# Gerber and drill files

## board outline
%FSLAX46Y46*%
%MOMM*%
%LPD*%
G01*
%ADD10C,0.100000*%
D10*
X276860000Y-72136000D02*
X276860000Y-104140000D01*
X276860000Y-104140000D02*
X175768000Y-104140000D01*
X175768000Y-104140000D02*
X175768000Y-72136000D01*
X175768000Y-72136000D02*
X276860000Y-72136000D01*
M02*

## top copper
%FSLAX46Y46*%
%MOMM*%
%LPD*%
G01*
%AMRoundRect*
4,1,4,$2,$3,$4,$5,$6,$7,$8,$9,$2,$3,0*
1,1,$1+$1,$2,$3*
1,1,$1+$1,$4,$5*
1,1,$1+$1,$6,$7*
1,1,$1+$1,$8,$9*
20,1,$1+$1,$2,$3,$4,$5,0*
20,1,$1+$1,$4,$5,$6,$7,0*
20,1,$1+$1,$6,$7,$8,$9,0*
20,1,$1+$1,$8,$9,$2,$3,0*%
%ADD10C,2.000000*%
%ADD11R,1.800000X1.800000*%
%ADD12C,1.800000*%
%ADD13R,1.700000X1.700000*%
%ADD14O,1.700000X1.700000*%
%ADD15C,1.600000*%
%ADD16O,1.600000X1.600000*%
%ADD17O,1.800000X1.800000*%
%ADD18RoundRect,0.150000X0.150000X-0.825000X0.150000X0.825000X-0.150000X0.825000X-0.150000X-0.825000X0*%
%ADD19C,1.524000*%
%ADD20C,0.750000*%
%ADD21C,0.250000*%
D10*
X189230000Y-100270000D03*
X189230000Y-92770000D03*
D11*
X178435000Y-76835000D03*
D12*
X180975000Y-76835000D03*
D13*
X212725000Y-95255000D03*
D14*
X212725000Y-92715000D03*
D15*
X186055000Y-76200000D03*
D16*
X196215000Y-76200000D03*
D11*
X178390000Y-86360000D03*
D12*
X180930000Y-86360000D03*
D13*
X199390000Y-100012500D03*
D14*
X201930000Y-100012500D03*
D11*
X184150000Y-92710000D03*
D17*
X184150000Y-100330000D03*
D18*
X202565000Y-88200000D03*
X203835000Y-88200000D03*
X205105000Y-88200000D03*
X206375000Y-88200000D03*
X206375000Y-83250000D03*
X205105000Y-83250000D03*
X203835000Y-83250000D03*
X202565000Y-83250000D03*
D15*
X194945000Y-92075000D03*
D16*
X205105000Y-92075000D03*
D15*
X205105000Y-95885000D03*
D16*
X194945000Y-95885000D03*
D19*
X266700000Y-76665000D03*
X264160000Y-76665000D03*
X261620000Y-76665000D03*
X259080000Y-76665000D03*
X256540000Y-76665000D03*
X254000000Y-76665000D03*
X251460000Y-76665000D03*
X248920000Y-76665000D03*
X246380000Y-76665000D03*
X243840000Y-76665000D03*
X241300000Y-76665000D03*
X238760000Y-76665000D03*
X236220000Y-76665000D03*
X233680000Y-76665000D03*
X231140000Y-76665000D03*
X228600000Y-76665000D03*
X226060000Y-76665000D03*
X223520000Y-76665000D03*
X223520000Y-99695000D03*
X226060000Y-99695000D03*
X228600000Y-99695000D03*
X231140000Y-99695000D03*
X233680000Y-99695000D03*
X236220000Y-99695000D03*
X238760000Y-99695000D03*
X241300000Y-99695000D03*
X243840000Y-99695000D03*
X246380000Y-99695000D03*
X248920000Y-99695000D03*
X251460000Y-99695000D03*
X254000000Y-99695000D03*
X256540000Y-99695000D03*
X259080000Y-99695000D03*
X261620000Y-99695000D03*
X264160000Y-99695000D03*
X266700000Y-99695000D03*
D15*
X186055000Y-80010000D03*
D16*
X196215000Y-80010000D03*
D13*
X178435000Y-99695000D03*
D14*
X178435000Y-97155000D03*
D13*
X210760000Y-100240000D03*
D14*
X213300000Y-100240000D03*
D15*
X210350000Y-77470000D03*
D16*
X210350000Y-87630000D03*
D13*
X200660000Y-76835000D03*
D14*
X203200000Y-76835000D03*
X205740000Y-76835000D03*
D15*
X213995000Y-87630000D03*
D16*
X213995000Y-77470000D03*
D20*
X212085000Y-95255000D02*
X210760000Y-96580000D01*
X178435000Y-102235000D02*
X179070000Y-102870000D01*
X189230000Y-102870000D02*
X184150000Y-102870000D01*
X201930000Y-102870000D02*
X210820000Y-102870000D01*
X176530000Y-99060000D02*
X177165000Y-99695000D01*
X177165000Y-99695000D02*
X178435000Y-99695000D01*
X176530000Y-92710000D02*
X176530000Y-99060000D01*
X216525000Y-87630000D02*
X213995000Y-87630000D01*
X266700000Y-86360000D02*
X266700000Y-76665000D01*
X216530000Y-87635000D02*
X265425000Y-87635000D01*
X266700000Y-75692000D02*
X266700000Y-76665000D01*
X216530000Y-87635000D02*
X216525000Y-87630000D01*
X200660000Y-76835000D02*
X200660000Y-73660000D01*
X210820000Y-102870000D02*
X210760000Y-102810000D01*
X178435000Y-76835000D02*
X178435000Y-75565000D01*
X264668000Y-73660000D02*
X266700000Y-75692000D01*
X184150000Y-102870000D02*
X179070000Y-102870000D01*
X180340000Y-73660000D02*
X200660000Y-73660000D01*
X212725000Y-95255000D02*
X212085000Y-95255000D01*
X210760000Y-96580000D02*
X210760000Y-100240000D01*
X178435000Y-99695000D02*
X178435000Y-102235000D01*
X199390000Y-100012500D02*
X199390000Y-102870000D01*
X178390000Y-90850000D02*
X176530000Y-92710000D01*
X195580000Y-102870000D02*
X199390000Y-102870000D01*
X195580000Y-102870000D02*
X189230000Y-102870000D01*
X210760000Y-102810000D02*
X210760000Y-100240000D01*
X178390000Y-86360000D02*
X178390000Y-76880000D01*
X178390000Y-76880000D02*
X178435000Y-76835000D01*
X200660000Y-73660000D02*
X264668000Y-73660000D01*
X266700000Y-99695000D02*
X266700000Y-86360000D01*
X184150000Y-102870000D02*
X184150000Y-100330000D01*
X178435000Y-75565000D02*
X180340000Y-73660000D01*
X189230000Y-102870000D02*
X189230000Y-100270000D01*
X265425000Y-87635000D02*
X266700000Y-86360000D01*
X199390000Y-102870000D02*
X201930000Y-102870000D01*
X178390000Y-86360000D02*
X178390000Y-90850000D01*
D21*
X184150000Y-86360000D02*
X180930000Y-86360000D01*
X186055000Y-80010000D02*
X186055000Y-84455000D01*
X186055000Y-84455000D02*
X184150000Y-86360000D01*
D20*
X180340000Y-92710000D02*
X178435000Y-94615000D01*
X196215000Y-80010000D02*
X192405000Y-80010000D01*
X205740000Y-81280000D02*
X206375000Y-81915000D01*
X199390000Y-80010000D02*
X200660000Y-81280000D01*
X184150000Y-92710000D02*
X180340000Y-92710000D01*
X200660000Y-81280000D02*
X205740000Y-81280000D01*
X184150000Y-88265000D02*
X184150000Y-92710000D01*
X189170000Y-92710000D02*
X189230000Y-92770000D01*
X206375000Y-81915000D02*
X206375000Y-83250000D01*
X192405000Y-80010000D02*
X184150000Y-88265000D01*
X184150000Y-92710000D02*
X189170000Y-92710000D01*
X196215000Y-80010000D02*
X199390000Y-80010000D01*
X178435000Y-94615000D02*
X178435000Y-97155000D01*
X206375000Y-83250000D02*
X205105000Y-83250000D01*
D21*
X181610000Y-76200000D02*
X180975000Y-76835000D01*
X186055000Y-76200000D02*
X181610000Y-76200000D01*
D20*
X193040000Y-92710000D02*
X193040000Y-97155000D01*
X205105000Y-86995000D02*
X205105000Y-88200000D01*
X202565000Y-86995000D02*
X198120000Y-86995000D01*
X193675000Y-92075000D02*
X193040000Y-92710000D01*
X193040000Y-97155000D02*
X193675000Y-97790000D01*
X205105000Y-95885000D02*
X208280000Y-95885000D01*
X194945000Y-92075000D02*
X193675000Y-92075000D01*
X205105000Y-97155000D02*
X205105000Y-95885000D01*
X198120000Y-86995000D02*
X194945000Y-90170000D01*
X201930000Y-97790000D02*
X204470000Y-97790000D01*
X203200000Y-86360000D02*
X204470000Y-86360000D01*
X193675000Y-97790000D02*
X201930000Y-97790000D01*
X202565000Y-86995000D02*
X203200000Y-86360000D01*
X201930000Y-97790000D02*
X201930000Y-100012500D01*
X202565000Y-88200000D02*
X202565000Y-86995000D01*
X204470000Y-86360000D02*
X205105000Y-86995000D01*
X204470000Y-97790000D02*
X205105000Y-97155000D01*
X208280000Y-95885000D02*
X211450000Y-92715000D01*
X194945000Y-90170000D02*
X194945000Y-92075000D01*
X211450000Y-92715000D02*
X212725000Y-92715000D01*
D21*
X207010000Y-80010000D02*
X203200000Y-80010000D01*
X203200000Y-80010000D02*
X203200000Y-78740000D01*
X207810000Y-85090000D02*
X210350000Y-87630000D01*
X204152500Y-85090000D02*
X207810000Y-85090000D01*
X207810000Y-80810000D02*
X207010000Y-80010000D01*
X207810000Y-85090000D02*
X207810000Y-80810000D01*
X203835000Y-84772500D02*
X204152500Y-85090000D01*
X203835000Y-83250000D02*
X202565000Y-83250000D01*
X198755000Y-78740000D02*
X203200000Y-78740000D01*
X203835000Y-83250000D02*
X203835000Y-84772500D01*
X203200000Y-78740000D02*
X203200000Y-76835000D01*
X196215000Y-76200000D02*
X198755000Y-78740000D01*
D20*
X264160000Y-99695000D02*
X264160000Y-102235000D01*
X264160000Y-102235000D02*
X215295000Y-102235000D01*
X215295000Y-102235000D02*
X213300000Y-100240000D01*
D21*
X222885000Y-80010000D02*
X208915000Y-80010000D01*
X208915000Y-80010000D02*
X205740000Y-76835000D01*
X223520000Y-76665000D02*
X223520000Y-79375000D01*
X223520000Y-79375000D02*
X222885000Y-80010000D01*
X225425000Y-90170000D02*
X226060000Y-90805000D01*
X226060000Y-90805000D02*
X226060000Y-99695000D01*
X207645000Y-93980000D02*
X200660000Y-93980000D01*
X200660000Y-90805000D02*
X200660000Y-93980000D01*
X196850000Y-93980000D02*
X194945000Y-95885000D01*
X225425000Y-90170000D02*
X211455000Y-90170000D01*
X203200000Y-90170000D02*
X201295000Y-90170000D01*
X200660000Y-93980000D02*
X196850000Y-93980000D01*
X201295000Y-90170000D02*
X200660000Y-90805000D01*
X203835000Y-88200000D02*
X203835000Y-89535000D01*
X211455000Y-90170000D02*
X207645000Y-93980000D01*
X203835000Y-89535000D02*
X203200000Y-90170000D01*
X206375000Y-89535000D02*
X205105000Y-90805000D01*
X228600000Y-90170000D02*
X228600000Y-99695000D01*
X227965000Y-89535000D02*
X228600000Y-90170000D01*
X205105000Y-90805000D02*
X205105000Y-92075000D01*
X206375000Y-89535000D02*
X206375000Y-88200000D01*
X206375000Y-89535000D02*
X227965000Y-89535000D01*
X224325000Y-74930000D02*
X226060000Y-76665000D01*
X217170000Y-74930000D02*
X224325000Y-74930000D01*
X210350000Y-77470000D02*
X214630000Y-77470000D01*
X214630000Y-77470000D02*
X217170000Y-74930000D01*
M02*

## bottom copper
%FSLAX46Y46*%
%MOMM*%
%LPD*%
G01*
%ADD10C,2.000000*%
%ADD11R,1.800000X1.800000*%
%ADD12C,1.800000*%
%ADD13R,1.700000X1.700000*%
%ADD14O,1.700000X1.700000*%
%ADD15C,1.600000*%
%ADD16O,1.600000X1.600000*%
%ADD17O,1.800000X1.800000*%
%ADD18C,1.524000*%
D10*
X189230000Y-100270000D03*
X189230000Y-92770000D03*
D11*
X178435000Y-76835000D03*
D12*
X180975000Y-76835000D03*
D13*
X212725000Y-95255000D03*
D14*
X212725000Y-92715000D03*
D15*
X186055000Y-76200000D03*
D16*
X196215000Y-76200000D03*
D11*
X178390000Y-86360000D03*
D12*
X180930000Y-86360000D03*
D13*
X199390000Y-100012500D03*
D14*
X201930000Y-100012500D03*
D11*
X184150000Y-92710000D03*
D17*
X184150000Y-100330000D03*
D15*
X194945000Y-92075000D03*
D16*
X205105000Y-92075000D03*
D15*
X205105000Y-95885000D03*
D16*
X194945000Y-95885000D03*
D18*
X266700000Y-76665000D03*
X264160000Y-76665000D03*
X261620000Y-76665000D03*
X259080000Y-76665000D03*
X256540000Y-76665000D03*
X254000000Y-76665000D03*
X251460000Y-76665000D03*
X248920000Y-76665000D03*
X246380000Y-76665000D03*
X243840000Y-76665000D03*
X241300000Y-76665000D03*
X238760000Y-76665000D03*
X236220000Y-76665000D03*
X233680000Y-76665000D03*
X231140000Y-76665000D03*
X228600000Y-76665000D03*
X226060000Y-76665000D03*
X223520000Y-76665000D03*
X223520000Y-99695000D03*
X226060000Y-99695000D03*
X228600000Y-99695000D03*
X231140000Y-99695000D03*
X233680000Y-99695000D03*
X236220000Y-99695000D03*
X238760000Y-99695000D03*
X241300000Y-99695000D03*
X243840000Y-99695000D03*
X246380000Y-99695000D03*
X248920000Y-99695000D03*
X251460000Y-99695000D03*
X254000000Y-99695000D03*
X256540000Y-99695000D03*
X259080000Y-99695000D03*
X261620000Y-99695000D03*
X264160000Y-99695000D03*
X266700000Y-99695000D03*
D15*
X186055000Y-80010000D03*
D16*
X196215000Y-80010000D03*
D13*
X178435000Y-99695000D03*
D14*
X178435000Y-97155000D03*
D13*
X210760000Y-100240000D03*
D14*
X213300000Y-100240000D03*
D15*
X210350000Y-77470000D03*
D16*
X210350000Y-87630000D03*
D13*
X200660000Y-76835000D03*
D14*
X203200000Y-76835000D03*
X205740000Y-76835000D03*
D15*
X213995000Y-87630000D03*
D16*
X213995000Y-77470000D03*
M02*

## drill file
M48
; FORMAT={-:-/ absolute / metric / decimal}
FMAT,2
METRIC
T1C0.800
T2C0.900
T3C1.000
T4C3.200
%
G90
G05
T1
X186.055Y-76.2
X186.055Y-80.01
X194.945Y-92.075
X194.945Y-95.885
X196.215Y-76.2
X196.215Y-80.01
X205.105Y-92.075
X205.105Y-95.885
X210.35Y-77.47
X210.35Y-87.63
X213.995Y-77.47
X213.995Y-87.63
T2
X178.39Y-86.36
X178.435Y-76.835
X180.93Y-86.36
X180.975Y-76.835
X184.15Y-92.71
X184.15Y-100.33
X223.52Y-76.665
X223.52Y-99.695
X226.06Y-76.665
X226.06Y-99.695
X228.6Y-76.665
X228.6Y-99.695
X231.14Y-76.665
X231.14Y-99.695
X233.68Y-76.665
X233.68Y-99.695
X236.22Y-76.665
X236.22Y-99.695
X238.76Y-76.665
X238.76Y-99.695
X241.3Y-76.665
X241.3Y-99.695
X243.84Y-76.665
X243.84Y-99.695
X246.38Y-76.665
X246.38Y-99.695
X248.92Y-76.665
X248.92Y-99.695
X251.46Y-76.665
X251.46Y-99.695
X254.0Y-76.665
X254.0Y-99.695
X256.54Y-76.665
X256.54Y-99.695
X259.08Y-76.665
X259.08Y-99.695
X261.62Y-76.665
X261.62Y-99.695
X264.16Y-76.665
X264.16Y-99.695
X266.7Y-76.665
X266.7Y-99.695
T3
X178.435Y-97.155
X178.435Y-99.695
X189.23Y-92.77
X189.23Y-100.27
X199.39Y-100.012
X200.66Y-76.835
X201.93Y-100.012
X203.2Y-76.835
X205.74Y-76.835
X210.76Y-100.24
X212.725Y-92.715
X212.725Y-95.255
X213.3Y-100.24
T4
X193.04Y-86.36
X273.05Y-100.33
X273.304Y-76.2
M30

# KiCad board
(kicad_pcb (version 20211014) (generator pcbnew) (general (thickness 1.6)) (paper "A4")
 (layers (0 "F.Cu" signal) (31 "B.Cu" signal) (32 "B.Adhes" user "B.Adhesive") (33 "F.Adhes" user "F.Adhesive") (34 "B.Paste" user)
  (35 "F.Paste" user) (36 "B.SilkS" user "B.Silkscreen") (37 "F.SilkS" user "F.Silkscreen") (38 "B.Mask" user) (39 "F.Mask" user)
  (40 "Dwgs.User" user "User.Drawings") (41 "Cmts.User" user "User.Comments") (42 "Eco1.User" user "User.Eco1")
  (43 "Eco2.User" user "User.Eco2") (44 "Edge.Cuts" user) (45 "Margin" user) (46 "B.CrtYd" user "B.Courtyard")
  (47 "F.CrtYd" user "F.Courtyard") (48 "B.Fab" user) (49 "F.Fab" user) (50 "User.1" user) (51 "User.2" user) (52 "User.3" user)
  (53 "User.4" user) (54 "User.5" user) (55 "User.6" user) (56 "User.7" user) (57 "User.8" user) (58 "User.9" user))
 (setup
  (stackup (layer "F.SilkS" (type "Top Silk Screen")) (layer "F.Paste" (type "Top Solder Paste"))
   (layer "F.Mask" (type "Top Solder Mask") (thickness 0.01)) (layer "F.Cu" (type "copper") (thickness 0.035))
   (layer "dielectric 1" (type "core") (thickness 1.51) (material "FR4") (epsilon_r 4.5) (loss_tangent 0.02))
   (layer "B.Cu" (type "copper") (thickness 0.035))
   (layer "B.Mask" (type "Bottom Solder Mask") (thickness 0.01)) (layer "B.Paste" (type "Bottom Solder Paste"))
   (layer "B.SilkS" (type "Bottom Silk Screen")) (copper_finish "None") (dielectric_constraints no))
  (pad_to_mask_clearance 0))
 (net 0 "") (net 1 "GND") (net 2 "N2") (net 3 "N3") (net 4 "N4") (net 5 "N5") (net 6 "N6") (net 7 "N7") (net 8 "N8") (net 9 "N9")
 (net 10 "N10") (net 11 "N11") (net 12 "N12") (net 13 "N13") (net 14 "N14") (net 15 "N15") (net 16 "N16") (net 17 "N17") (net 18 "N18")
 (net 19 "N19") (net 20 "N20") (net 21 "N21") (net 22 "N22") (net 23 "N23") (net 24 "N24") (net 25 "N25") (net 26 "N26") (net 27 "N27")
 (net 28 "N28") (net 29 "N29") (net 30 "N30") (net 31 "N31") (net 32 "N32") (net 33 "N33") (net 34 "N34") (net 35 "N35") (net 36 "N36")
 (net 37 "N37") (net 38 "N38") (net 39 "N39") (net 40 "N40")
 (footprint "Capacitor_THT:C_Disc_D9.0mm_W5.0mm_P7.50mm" (layer "F.Cu") (at 189.23 100.27 90)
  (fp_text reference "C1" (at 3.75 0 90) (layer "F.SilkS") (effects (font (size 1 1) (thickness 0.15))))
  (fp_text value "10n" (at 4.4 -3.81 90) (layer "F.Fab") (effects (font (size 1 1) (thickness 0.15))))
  (pad "1" thru_hole circle (at 0 0 90) (size 2 2) (drill 1) (layers *.Cu *.Mask) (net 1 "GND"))
  (pad "2" thru_hole circle (at 7.5 0 90) (size 2 2) (drill 1) (layers *.Cu *.Mask) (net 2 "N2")))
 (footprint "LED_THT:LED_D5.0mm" (layer "F.Cu") (at 178.435 76.835)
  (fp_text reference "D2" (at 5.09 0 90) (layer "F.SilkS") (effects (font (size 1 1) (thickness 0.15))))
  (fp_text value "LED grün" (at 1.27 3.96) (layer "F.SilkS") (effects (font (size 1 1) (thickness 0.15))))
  (pad "1" thru_hole rect (at 0 0) (size 1.8 1.8) (drill 0.9) (layers *.Cu *.Mask) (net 1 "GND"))
  (pad "2" thru_hole circle (at 2.54 0) (size 1.8 1.8) (drill 0.9) (layers *.Cu *.Mask) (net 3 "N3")))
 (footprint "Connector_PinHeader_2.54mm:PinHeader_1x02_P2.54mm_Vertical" (layer "F.Cu") (at 212.725 95.255 180)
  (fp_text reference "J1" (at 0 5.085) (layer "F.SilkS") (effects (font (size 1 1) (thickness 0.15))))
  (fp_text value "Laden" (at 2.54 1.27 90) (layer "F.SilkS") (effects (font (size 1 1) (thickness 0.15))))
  (pad "1" thru_hole rect (at 0 0 180) (size 1.7 1.7) (drill 1) (layers *.Cu *.Mask) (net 1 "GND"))
  (pad "2" thru_hole oval (at 0 2.54 180) (size 1.7 1.7) (drill 1) (layers *.Cu *.Mask) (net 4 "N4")))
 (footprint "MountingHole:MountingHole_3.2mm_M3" (layer "F.Cu") (at 193.04 86.36)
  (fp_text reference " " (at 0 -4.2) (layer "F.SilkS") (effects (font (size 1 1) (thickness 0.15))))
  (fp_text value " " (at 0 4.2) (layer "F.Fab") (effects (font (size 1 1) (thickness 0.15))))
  (pad "" np_thru_hole circle (at 0 0) (size 3.2 3.2) (drill 3.2) (layers *.Cu *.Mask)))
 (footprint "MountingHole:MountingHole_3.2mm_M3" (layer "F.Cu") (at 273.05 100.33)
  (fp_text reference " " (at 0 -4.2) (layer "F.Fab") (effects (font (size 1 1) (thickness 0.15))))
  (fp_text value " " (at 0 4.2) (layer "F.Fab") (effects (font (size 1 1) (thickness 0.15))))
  (pad "" np_thru_hole circle (at 0 0) (size 3.2 3.2) (drill 3.2) (layers *.Cu *.Mask)))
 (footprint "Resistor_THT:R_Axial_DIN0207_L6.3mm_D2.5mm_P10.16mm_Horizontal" (layer "F.Cu") (at 186.055 76.2)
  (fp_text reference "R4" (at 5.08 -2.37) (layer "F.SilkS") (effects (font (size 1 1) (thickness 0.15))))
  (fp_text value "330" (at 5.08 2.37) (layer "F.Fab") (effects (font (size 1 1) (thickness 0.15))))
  (pad "1" thru_hole circle (at 0 0) (size 1.6 1.6) (drill 0.8) (layers *.Cu *.Mask) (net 3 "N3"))
  (pad "2" thru_hole oval (at 10.16 0) (size 1.6 1.6) (drill 0.8) (layers *.Cu *.Mask) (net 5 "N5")))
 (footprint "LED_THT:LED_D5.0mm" (layer "F.Cu") (at 178.39 86.36)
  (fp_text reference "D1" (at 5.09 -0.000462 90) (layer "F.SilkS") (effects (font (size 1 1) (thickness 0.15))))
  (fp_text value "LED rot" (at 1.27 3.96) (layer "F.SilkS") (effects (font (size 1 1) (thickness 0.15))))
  (pad "1" thru_hole rect (at 0 0) (size 1.8 1.8) (drill 0.9) (layers *.Cu *.Mask) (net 1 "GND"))
  (pad "2" thru_hole circle (at 2.54 0) (size 1.8 1.8) (drill 0.9) (layers *.Cu *.Mask) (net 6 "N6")))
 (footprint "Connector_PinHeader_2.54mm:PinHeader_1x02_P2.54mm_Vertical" (layer "F.Cu") (at 199.39 100.0125 90)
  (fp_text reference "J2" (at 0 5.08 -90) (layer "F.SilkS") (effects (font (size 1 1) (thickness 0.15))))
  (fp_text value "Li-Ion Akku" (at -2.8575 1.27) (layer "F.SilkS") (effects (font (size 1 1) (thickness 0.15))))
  (pad "1" thru_hole rect (at 0 0 90) (size 1.7 1.7) (drill 1) (layers *.Cu *.Mask) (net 1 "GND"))
  (pad "2" thru_hole oval (at 0 2.54 90) (size 1.7 1.7) (drill 1) (layers *.Cu *.Mask) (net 4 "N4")))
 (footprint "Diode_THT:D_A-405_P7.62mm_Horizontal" (layer "F.Cu") (at 184.15 92.71 -90)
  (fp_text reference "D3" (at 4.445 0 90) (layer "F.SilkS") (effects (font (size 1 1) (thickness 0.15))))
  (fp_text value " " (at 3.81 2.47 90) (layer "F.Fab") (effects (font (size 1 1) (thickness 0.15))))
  (pad "1" thru_hole rect (at 0 0 270) (size 1.8 1.8) (drill 0.9) (layers *.Cu *.Mask) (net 2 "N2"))
  (pad "2" thru_hole oval (at 7.62 0 270) (size 1.8 1.8) (drill 0.9) (layers *.Cu *.Mask) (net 1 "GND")))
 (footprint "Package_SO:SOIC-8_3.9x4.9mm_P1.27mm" (layer "F.Cu") (at 204.47 85.725 90)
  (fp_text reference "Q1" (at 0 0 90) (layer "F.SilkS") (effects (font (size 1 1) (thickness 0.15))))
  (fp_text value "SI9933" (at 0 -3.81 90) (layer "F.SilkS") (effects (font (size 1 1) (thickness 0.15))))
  (pad "1" smd roundrect (at -2.475 -1.905 90) (size 1.95 0.6) (layers "F.Cu" "F.Paste" "F.Mask") (roundrect_rratio 0.25) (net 4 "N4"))
  (pad "2" smd roundrect (at -2.475 -0.635 90) (size 1.95 0.6) (layers "F.Cu" "F.Paste" "F.Mask") (roundrect_rratio 0.25) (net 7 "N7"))
  (pad "3" smd roundrect (at -2.475 0.635 90) (size 1.95 0.6) (layers "F.Cu" "F.Paste" "F.Mask") (roundrect_rratio 0.25) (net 4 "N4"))
  (pad "4" smd roundrect (at -2.475 1.905 90) (size 1.95 0.6) (layers "F.Cu" "F.Paste" "F.Mask") (roundrect_rratio 0.25) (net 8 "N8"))
  (pad "5" smd roundrect (at 2.475 1.905 90) (size 1.95 0.6) (layers "F.Cu" "F.Paste" "F.Mask") (roundrect_rratio 0.25) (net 2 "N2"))
  (pad "6" smd roundrect (at 2.475 0.635 90) (size 1.95 0.6) (layers "F.Cu" "F.Paste" "F.Mask") (roundrect_rratio 0.25) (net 2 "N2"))
  (pad "7" smd roundrect (at 2.475 -0.635 90) (size 1.95 0.6) (layers "F.Cu" "F.Paste" "F.Mask") (roundrect_rratio 0.25) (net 5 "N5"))
  (pad "8" smd roundrect (at 2.475 -1.905 90) (size 1.95 0.6) (layers "F.Cu" "F.Paste" "F.Mask") (roundrect_rratio 0.25) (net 5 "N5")))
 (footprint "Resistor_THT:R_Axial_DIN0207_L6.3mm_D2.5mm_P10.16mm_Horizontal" (layer "F.Cu") (at 194.945 92.075)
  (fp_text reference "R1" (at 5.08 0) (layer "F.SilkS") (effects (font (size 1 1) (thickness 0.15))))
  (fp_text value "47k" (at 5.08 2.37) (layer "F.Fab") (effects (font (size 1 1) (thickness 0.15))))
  (pad "1" thru_hole circle (at 0 0) (size 1.6 1.6) (drill 0.8) (layers *.Cu *.Mask) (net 4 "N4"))
  (pad "2" thru_hole oval (at 10.16 0) (size 1.6 1.6) (drill 0.8) (layers *.Cu *.Mask) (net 8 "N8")))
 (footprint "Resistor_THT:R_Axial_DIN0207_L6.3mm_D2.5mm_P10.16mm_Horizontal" (layer "F.Cu") (at 205.105 95.885 180)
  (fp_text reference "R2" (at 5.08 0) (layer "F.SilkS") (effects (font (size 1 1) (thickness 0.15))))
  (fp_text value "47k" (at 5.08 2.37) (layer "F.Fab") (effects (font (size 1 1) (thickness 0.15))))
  (pad "1" thru_hole circle (at 0 0 180) (size 1.6 1.6) (drill 0.8) (layers *.Cu *.Mask) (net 4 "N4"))
  (pad "2" thru_hole oval (at 10.16 0 180) (size 1.6 1.6) (drill 0.8) (layers *.Cu *.Mask) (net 7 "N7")))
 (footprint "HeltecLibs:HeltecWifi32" (layer "F.Cu") (at 241.3 88.18 -90)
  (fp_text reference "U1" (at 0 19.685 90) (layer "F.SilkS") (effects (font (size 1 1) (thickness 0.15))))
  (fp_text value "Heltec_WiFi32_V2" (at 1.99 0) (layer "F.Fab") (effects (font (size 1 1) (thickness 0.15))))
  (pad "1" thru_hole circle (at -11.515 -25.4 270) (size 1.524 1.524) (drill 0.9) (layers *.Cu *.Mask) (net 1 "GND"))
  (pad "2" thru_hole circle (at -11.515 -22.86 270) (size 1.524 1.524) (drill 0.9) (layers *.Cu *.Mask) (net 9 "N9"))
  (pad "3" thru_hole circle (at -11.515 -20.32 270) (size 1.524 1.524) (drill 0.9) (layers *.Cu *.Mask) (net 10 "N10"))
  (pad "4" thru_hole circle (at -11.515 -17.78 270) (size 1.524 1.524) (drill 0.9) (layers *.Cu *.Mask) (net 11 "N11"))
  (pad "5" thru_hole circle (at -11.515 -15.24 270) (size 1.524 1.524) (drill 0.9) (layers *.Cu *.Mask) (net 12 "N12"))
  (pad "6" thru_hole circle (at -11.515 -12.7 270) (size 1.524 1.524) (drill 0.9) (layers *.Cu *.Mask) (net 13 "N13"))
  (pad "7" thru_hole circle (at -11.515 -10.16 270) (size 1.524 1.524) (drill 0.9) (layers *.Cu *.Mask) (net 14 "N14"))
  (pad "8" thru_hole circle (at -11.515 -7.62 270) (size 1.524 1.524) (drill 0.9) (layers *.Cu *.Mask) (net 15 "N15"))
  (pad "9" thru_hole circle (at -11.515 -5.08 270) (size 1.524 1.524) (drill 0.9) (layers *.Cu *.Mask) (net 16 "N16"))
  (pad "10" thru_hole circle (at -11.515 -2.54 270) (size 1.524 1.524) (drill 0.9) (layers *.Cu *.Mask) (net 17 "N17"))
  (pad "11" thru_hole circle (at -11.515 0 270) (size 1.524 1.524) (drill 0.9) (layers *.Cu *.Mask) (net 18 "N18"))
  (pad "12" thru_hole circle (at -11.515 2.54 270) (size 1.524 1.524) (drill 0.9) (layers *.Cu *.Mask) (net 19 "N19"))
  (pad "13" thru_hole circle (at -11.515 5.08 270) (size 1.524 1.524) (drill 0.9) (layers *.Cu *.Mask) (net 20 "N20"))
  (pad "14" thru_hole circle (at -11.515 7.62 270) (size 1.524 1.524) (drill 0.9) (layers *.Cu *.Mask) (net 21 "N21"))
  (pad "15" thru_hole circle (at -11.515 10.16 270) (size 1.524 1.524) (drill 0.9) (layers *.Cu *.Mask) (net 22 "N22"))
  (pad "16" thru_hole circle (at -11.515 12.7 270) (size 1.524 1.524) (drill 0.9) (layers *.Cu *.Mask) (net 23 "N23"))
  (pad "17" thru_hole circle (at -11.515 15.24 270) (size 1.524 1.524) (drill 0.9) (layers *.Cu *.Mask) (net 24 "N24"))
  (pad "18" thru_hole circle (at -11.515 17.78 270) (size 1.524 1.524) (drill 0.9) (layers *.Cu *.Mask) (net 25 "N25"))
  (pad "19" thru_hole circle (at 11.515 17.78 270) (size 1.524 1.524) (drill 0.9) (layers *.Cu *.Mask) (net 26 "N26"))
  (pad "20" thru_hole circle (at 11.515 15.24 270) (size 1.524 1.524) (drill 0.9) (layers *.Cu *.Mask) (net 7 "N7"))
  (pad "21" thru_hole circle (at 11.515 12.7 270) (size 1.524 1.524) (drill 0.9) (layers *.Cu *.Mask) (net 8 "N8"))
  (pad "22" thru_hole circle (at 11.515 10.16 270) (size 1.524 1.524) (drill 0.9) (layers *.Cu *.Mask) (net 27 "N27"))
  (pad "23" thru_hole circle (at 11.515 7.62 270) (size 1.524 1.524) (drill 0.9) (layers *.Cu *.Mask) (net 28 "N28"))
  (pad "24" thru_hole circle (at 11.515 5.08 270) (size 1.524 1.524) (drill 0.9) (layers *.Cu *.Mask) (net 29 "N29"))
  (pad "25" thru_hole circle (at 11.515 2.54 270) (size 1.524 1.524) (drill 0.9) (layers *.Cu *.Mask) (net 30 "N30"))
  (pad "26" thru_hole circle (at 11.515 0 270) (size 1.524 1.524) (drill 0.9) (layers *.Cu *.Mask) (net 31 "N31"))
  (pad "27" thru_hole circle (at 11.515 -2.54 270) (size 1.524 1.524) (drill 0.9) (layers *.Cu *.Mask) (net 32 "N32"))
  (pad "28" thru_hole circle (at 11.515 -5.08 270) (size 1.524 1.524) (drill 0.9) (layers *.Cu *.Mask) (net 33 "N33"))
  (pad "29" thru_hole circle (at 11.515 -7.62 270) (size 1.524 1.524) (drill 0.9) (layers *.Cu *.Mask) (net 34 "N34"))
  (pad "30" thru_hole circle (at 11.515 -10.16 270) (size 1.524 1.524) (drill 0.9) (layers *.Cu *.Mask) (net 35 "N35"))
  (pad "31" thru_hole circle (at 11.515 -12.7 270) (size 1.524 1.524) (drill 0.9) (layers *.Cu *.Mask) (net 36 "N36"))
  (pad "32" thru_hole circle (at 11.515 -15.24 270) (size 1.524 1.524) (drill 0.9) (layers *.Cu *.Mask) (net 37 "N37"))
  (pad "33" thru_hole circle (at 11.515 -17.78 270) (size 1.524 1.524) (drill 0.9) (layers *.Cu *.Mask) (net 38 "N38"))
  (pad "34" thru_hole circle (at 11.515 -20.32 270) (size 1.524 1.524) (drill 0.9) (layers *.Cu *.Mask) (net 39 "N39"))
  (pad "35" thru_hole circle (at 11.515 -22.86 270) (size 1.524 1.524) (drill 0.9) (layers *.Cu *.Mask) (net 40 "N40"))
  (pad "36" thru_hole circle (at 11.515 -25.4 270) (size 1.524 1.524) (drill 0.9) (layers *.Cu *.Mask) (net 1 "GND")))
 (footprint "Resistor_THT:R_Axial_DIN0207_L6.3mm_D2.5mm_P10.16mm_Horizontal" (layer "F.Cu") (at 186.055 80.01)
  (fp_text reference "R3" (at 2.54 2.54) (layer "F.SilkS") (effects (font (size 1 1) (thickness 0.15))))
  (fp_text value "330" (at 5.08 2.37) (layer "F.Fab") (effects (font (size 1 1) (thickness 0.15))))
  (pad "1" thru_hole circle (at 0 0) (size 1.6 1.6) (drill 0.8) (layers *.Cu *.Mask) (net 6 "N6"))
  (pad "2" thru_hole oval (at 10.16 0) (size 1.6 1.6) (drill 0.8) (layers *.Cu *.Mask) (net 2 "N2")))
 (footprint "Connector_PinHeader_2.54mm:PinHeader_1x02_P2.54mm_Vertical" (layer "F.Cu") (at 178.435 99.695 180)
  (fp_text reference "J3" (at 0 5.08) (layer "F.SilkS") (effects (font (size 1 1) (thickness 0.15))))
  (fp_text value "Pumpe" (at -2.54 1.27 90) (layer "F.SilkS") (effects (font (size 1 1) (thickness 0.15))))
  (pad "1" thru_hole rect (at 0 0 180) (size 1.7 1.7) (drill 1) (layers *.Cu *.Mask) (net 1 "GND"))
  (pad "2" thru_hole oval (at 0 2.54 180) (size 1.7 1.7) (drill 1) (layers *.Cu *.Mask) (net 2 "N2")))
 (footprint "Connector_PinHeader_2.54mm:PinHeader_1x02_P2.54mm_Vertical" (layer "F.Cu") (at 210.76 100.24 90)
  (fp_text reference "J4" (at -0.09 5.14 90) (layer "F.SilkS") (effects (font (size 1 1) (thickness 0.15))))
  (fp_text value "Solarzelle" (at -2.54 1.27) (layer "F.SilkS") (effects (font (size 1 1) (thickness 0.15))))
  (pad "1" thru_hole rect (at 0 0 90) (size 1.7 1.7) (drill 1) (layers *.Cu *.Mask) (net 1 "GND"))
  (pad "2" thru_hole oval (at 0 2.54 90) (size 1.7 1.7) (drill 1) (layers *.Cu *.Mask) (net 40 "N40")))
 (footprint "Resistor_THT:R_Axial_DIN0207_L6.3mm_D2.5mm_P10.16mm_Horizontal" (layer "F.Cu") (at 210.35 77.47 -90)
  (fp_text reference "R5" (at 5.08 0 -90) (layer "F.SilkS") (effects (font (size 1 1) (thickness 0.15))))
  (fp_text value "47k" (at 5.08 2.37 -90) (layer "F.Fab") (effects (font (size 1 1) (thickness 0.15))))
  (pad "1" thru_hole circle (at 0 0 270) (size 1.6 1.6) (drill 0.8) (layers *.Cu *.Mask) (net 24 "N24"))
  (pad "2" thru_hole oval (at 10.16 0 270) (size 1.6 1.6) (drill 0.8) (layers *.Cu *.Mask) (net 5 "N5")))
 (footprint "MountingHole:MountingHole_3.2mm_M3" (layer "F.Cu") (at 273.304 76.2)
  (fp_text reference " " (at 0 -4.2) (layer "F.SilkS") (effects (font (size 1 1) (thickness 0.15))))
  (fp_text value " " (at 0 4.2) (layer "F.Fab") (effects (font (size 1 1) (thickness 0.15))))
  (pad "" np_thru_hole circle (at 0 0) (size 3.2 3.2) (drill 3.2) (layers *.Cu *.Mask)))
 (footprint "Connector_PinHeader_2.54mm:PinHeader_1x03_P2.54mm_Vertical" (layer "F.Cu") (at 200.66 76.835 90)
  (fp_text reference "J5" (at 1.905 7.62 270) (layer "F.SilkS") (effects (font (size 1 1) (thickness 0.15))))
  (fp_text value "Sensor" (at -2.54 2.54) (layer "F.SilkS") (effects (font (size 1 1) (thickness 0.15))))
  (pad "1" thru_hole rect (at 0 0 90) (size 1.7 1.7) (drill 1) (layers *.Cu *.Mask) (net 1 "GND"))
  (pad "2" thru_hole oval (at 0 2.54 90) (size 1.7 1.7) (drill 1) (layers *.Cu *.Mask) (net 5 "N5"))
  (pad "3" thru_hole oval (at 0 5.08 90) (size 1.7 1.7) (drill 1) (layers *.Cu *.Mask) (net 25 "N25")))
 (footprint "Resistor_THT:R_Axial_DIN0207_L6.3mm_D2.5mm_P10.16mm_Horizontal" (layer "F.Cu") (at 213.995 87.63 90)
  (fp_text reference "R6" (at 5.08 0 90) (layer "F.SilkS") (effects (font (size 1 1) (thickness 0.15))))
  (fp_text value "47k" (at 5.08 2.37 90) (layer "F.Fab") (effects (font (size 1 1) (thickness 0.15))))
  (pad "1" thru_hole circle (at 0 0 90) (size 1.6 1.6) (drill 0.8) (layers *.Cu *.Mask) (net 1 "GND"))
  (pad "2" thru_hole oval (at 10.16 0 90) (size 1.6 1.6) (drill 0.8) (layers *.Cu *.Mask) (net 24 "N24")))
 (gr_line (start 276.86 72.136) (end 276.86 104.14) (layer "Edge.Cuts") (width 0.1))
 (gr_line (start 276.86 104.14) (end 175.768 104.14) (layer "Edge.Cuts") (width 0.1))
 (gr_line (start 175.768 104.14) (end 175.768 72.136) (layer "Edge.Cuts") (width 0.1))
 (gr_line (start 175.768 72.136) (end 276.86 72.136) (layer "Edge.Cuts") (width 0.1))
 (segment (start 212.085 95.255) (end 210.76 96.58) (width 0.75) (layer "F.Cu") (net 1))
 (segment (start 178.435 102.235) (end 179.07 102.87) (width 0.75) (layer "F.Cu") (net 1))
 (segment (start 189.23 102.87) (end 184.15 102.87) (width 0.75) (layer "F.Cu") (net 1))
 (segment (start 201.93 102.87) (end 210.82 102.87) (width 0.75) (layer "F.Cu") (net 1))
 (segment (start 176.53 99.06) (end 177.165 99.695) (width 0.75) (layer "F.Cu") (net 1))
 (segment (start 177.165 99.695) (end 178.435 99.695) (width 0.75) (layer "F.Cu") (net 1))
 (segment (start 176.53 92.71) (end 176.53 99.06) (width 0.75) (layer "F.Cu") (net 1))
 (segment (start 216.525 87.63) (end 213.995 87.63) (width 0.75) (layer "F.Cu") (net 1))
 (segment (start 266.7 86.36) (end 266.7 76.665) (width 0.75) (layer "F.Cu") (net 1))
 (segment (start 216.53 87.635) (end 265.425 87.635) (width 0.75) (layer "F.Cu") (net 1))
 (segment (start 266.7 75.692) (end 266.7 76.665) (width 0.75) (layer "F.Cu") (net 1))
 (segment (start 216.53 87.635) (end 216.525 87.63) (width 0.75) (layer "F.Cu") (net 1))
 (segment (start 200.66 76.835) (end 200.66 73.66) (width 0.75) (layer "F.Cu") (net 1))
 (segment (start 210.82 102.87) (end 210.76 102.81) (width 0.75) (layer "F.Cu") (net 1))
 (segment (start 178.435 76.835) (end 178.435 75.565) (width 0.75) (layer "F.Cu") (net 1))
 (segment (start 264.668 73.66) (end 266.7 75.692) (width 0.75) (layer "F.Cu") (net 1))
 (segment (start 184.15 102.87) (end 179.07 102.87) (width 0.75) (layer "F.Cu") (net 1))
 (segment (start 180.34 73.66) (end 200.66 73.66) (width 0.75) (layer "F.Cu") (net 1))
 (segment (start 212.725 95.255) (end 212.085 95.255) (width 0.75) (layer "F.Cu") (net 1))
 (segment (start 210.76 96.58) (end 210.76 100.24) (width 0.75) (layer "F.Cu") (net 1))
 (segment (start 178.435 99.695) (end 178.435 102.235) (width 0.75) (layer "F.Cu") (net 1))
 (segment (start 199.39 100.0125) (end 199.39 102.87) (width 0.75) (layer "F.Cu") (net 1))
 (segment (start 178.39 90.85) (end 176.53 92.71) (width 0.75) (layer "F.Cu") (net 1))
 (segment (start 195.58 102.87) (end 199.39 102.87) (width 0.75) (layer "F.Cu") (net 1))
 (segment (start 195.58 102.87) (end 189.23 102.87) (width 0.75) (layer "F.Cu") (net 1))
 (segment (start 210.76 102.81) (end 210.76 100.24) (width 0.75) (layer "F.Cu") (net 1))
 (segment (start 178.39 86.36) (end 178.39 76.88) (width 0.75) (layer "F.Cu") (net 1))
 (segment (start 178.39 76.88) (end 178.435 76.835) (width 0.75) (layer "F.Cu") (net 1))
 (segment (start 200.66 73.66) (end 264.668 73.66) (width 0.75) (layer "F.Cu") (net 1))
 (segment (start 266.7 99.695) (end 266.7 86.36) (width 0.75) (layer "F.Cu") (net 1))
 (segment (start 184.15 102.87) (end 184.15 100.33) (width 0.75) (layer "F.Cu") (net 1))
 (segment (start 178.435 75.565) (end 180.34 73.66) (width 0.75) (layer "F.Cu") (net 1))
 (segment (start 189.23 102.87) (end 189.23 100.27) (width 0.75) (layer "F.Cu") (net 1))
 (segment (start 265.425 87.635) (end 266.7 86.36) (width 0.75) (layer "F.Cu") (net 1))
 (segment (start 199.39 102.87) (end 201.93 102.87) (width 0.75) (layer "F.Cu") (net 1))
 (segment (start 178.39 86.36) (end 178.39 90.85) (width 0.75) (layer "F.Cu") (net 1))
 (segment (start 184.15 86.36) (end 180.93 86.36) (width 0.25) (layer "F.Cu") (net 6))
 (segment (start 186.055 80.01) (end 186.055 84.455) (width 0.25) (layer "F.Cu") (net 6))
 (segment (start 186.055 84.455) (end 184.15 86.36) (width 0.25) (layer "F.Cu") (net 6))
 (segment (start 180.34 92.71) (end 178.435 94.615) (width 0.75) (layer "F.Cu") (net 2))
 (segment (start 196.215 80.01) (end 192.405 80.01) (width 0.75) (layer "F.Cu") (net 2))
 (segment (start 205.74 81.28) (end 206.375 81.915) (width 0.75) (layer "F.Cu") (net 2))
 (segment (start 199.39 80.01) (end 200.66 81.28) (width 0.75) (layer "F.Cu") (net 2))
 (segment (start 184.15 92.71) (end 180.34 92.71) (width 0.75) (layer "F.Cu") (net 2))
 (segment (start 200.66 81.28) (end 205.74 81.28) (width 0.75) (layer "F.Cu") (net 2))
 (segment (start 184.15 88.265) (end 184.15 92.71) (width 0.75) (layer "F.Cu") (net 2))
 (segment (start 189.17 92.71) (end 189.23 92.77) (width 0.75) (layer "F.Cu") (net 2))
 (segment (start 206.375 81.915) (end 206.375 83.25) (width 0.75) (layer "F.Cu") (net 2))
 (segment (start 192.405 80.01) (end 184.15 88.265) (width 0.75) (layer "F.Cu") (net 2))
 (segment (start 184.15 92.71) (end 189.17 92.71) (width 0.75) (layer "F.Cu") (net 2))
 (segment (start 196.215 80.01) (end 199.39 80.01) (width 0.75) (layer "F.Cu") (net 2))
 (segment (start 178.435 94.615) (end 178.435 97.155) (width 0.75) (layer "F.Cu") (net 2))
 (segment (start 206.375 83.25) (end 205.105 83.25) (width 0.75) (layer "F.Cu") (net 2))
 (segment (start 181.61 76.2) (end 180.975 76.835) (width 0.25) (layer "F.Cu") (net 3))
 (segment (start 186.055 76.2) (end 181.61 76.2) (width 0.25) (layer "F.Cu") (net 3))
 (segment (start 193.04 92.71) (end 193.04 97.155) (width 0.75) (layer "F.Cu") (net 4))
 (segment (start 205.105 86.995) (end 205.105 88.2) (width 0.75) (layer "F.Cu") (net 4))
 (segment (start 202.565 86.995) (end 198.12 86.995) (width 0.75) (layer "F.Cu") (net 4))
 (segment (start 193.675 92.075) (end 193.04 92.71) (width 0.75) (layer "F.Cu") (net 4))
 (segment (start 193.04 97.155) (end 193.675 97.79) (width 0.75) (layer "F.Cu") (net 4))
 (segment (start 205.105 95.885) (end 208.28 95.885) (width 0.75) (layer "F.Cu") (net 4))
 (segment (start 194.945 92.075) (end 193.675 92.075) (width 0.75) (layer "F.Cu") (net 4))
 (segment (start 205.105 97.155) (end 205.105 95.885) (width 0.75) (layer "F.Cu") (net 4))
 (segment (start 198.12 86.995) (end 194.945 90.17) (width 0.75) (layer "F.Cu") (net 4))
 (segment (start 201.93 97.79) (end 204.47 97.79) (width 0.75) (layer "F.Cu") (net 4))
 (segment (start 203.2 86.36) (end 204.47 86.36) (width 0.75) (layer "F.Cu") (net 4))
 (segment (start 193.675 97.79) (end 201.93 97.79) (width 0.75) (layer "F.Cu") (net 4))
 (segment (start 202.565 86.995) (end 203.2 86.36) (width 0.75) (layer "F.Cu") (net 4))
 (segment (start 201.93 97.79) (end 201.93 100.0125) (width 0.75) (layer "F.Cu") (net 4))
 (segment (start 202.565 88.2) (end 202.565 86.995) (width 0.75) (layer "F.Cu") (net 4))
 (segment (start 204.47 86.36) (end 205.105 86.995) (width 0.75) (layer "F.Cu") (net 4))
 (segment (start 204.47 97.79) (end 205.105 97.155) (width 0.75) (layer "F.Cu") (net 4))
 (segment (start 208.28 95.885) (end 211.45 92.715) (width 0.75) (layer "F.Cu") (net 4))
 (segment (start 194.945 90.17) (end 194.945 92.075) (width 0.75) (layer "F.Cu") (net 4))
 (segment (start 211.45 92.715) (end 212.725 92.715) (width 0.75) (layer "F.Cu") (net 4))
 (segment (start 207.01 80.01) (end 203.2 80.01) (width 0.25) (layer "F.Cu") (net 5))
 (segment (start 203.2 80.01) (end 203.2 78.74) (width 0.25) (layer "F.Cu") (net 5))
 (segment (start 207.81 85.09) (end 210.35 87.63) (width 0.25) (layer "F.Cu") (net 5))
 (segment (start 204.1525 85.09) (end 207.81 85.09) (width 0.25) (layer "F.Cu") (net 5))
 (segment (start 207.81 80.81) (end 207.01 80.01) (width 0.25) (layer "F.Cu") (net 5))
 (segment (start 207.81 85.09) (end 207.81 80.81) (width 0.25) (layer "F.Cu") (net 5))
 (segment (start 203.835 84.7725) (end 204.1525 85.09) (width 0.25) (layer "F.Cu") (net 5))
 (segment (start 203.835 83.25) (end 202.565 83.25) (width 0.25) (layer "F.Cu") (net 5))
 (segment (start 198.755 78.74) (end 203.2 78.74) (width 0.25) (layer "F.Cu") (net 5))
 (segment (start 203.835 83.25) (end 203.835 84.7725) (width 0.25) (layer "F.Cu") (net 5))
 (segment (start 203.2 78.74) (end 203.2 76.835) (width 0.25) (layer "F.Cu") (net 5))
 (segment (start 196.215 76.2) (end 198.755 78.74) (width 0.25) (layer "F.Cu") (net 5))
 (segment (start 264.16 99.695) (end 264.16 102.235) (width 0.75) (layer "F.Cu") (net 40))
 (segment (start 264.16 102.235) (end 215.295 102.235) (width 0.75) (layer "F.Cu") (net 40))
 (segment (start 215.295 102.235) (end 213.3 100.24) (width 0.75) (layer "F.Cu") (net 40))
 (segment (start 222.885 80.01) (end 208.915 80.01) (width 0.25) (layer "F.Cu") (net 25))
 (segment (start 208.915 80.01) (end 205.74 76.835) (width 0.25) (layer "F.Cu") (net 25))
 (segment (start 223.52 76.665) (end 223.52 79.375) (width 0.25) (layer "F.Cu") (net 25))
 (segment (start 223.52 79.375) (end 222.885 80.01) (width 0.25) (layer "F.Cu") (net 25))
 (segment (start 225.425 90.17) (end 226.06 90.805) (width 0.25) (layer "F.Cu") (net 7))
 (segment (start 226.06 90.805) (end 226.06 99.695) (width 0.25) (layer "F.Cu") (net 7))
 (segment (start 207.645 93.98) (end 200.66 93.98) (width 0.25) (layer "F.Cu") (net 7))
 (segment (start 200.66 90.805) (end 200.66 93.98) (width 0.25) (layer "F.Cu") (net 7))
 (segment (start 196.85 93.98) (end 194.945 95.885) (width 0.25) (layer "F.Cu") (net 7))
 (segment (start 225.425 90.17) (end 211.455 90.17) (width 0.25) (layer "F.Cu") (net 7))
 (segment (start 203.2 90.17) (end 201.295 90.17) (width 0.25) (layer "F.Cu") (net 7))
 (segment (start 200.66 93.98) (end 196.85 93.98) (width 0.25) (layer "F.Cu") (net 7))
 (segment (start 201.295 90.17) (end 200.66 90.805) (width 0.25) (layer "F.Cu") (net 7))
 (segment (start 203.835 88.2) (end 203.835 89.535) (width 0.25) (layer "F.Cu") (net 7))
 (segment (start 211.455 90.17) (end 207.645 93.98) (width 0.25) (layer "F.Cu") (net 7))
 (segment (start 203.835 89.535) (end 203.2 90.17) (width 0.25) (layer "F.Cu") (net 7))
 (segment (start 206.375 89.535) (end 205.105 90.805) (width 0.25) (layer "F.Cu") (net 8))
 (segment (start 228.6 90.17) (end 228.6 99.695) (width 0.25) (layer "F.Cu") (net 8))
 (segment (start 227.965 89.535) (end 228.6 90.17) (width 0.25) (layer "F.Cu") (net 8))
 (segment (start 205.105 90.805) (end 205.105 92.075) (width 0.25) (layer "F.Cu") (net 8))
 (segment (start 206.375 89.535) (end 206.375 88.2) (width 0.25) (layer "F.Cu") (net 8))
 (segment (start 206.375 89.535) (end 227.965 89.535) (width 0.25) (layer "F.Cu") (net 8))
 (segment (start 224.325 74.93) (end 226.06 76.665) (width 0.25) (layer "F.Cu") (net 24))
 (segment (start 217.17 74.93) (end 224.325 74.93) (width 0.25) (layer "F.Cu") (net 24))
 (segment (start 210.35 77.47) (end 214.63 77.47) (width 0.25) (layer "F.Cu") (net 24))
 (segment (start 214.63 77.47) (end 217.17 74.93) (width 0.25) (layer "F.Cu") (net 24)))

